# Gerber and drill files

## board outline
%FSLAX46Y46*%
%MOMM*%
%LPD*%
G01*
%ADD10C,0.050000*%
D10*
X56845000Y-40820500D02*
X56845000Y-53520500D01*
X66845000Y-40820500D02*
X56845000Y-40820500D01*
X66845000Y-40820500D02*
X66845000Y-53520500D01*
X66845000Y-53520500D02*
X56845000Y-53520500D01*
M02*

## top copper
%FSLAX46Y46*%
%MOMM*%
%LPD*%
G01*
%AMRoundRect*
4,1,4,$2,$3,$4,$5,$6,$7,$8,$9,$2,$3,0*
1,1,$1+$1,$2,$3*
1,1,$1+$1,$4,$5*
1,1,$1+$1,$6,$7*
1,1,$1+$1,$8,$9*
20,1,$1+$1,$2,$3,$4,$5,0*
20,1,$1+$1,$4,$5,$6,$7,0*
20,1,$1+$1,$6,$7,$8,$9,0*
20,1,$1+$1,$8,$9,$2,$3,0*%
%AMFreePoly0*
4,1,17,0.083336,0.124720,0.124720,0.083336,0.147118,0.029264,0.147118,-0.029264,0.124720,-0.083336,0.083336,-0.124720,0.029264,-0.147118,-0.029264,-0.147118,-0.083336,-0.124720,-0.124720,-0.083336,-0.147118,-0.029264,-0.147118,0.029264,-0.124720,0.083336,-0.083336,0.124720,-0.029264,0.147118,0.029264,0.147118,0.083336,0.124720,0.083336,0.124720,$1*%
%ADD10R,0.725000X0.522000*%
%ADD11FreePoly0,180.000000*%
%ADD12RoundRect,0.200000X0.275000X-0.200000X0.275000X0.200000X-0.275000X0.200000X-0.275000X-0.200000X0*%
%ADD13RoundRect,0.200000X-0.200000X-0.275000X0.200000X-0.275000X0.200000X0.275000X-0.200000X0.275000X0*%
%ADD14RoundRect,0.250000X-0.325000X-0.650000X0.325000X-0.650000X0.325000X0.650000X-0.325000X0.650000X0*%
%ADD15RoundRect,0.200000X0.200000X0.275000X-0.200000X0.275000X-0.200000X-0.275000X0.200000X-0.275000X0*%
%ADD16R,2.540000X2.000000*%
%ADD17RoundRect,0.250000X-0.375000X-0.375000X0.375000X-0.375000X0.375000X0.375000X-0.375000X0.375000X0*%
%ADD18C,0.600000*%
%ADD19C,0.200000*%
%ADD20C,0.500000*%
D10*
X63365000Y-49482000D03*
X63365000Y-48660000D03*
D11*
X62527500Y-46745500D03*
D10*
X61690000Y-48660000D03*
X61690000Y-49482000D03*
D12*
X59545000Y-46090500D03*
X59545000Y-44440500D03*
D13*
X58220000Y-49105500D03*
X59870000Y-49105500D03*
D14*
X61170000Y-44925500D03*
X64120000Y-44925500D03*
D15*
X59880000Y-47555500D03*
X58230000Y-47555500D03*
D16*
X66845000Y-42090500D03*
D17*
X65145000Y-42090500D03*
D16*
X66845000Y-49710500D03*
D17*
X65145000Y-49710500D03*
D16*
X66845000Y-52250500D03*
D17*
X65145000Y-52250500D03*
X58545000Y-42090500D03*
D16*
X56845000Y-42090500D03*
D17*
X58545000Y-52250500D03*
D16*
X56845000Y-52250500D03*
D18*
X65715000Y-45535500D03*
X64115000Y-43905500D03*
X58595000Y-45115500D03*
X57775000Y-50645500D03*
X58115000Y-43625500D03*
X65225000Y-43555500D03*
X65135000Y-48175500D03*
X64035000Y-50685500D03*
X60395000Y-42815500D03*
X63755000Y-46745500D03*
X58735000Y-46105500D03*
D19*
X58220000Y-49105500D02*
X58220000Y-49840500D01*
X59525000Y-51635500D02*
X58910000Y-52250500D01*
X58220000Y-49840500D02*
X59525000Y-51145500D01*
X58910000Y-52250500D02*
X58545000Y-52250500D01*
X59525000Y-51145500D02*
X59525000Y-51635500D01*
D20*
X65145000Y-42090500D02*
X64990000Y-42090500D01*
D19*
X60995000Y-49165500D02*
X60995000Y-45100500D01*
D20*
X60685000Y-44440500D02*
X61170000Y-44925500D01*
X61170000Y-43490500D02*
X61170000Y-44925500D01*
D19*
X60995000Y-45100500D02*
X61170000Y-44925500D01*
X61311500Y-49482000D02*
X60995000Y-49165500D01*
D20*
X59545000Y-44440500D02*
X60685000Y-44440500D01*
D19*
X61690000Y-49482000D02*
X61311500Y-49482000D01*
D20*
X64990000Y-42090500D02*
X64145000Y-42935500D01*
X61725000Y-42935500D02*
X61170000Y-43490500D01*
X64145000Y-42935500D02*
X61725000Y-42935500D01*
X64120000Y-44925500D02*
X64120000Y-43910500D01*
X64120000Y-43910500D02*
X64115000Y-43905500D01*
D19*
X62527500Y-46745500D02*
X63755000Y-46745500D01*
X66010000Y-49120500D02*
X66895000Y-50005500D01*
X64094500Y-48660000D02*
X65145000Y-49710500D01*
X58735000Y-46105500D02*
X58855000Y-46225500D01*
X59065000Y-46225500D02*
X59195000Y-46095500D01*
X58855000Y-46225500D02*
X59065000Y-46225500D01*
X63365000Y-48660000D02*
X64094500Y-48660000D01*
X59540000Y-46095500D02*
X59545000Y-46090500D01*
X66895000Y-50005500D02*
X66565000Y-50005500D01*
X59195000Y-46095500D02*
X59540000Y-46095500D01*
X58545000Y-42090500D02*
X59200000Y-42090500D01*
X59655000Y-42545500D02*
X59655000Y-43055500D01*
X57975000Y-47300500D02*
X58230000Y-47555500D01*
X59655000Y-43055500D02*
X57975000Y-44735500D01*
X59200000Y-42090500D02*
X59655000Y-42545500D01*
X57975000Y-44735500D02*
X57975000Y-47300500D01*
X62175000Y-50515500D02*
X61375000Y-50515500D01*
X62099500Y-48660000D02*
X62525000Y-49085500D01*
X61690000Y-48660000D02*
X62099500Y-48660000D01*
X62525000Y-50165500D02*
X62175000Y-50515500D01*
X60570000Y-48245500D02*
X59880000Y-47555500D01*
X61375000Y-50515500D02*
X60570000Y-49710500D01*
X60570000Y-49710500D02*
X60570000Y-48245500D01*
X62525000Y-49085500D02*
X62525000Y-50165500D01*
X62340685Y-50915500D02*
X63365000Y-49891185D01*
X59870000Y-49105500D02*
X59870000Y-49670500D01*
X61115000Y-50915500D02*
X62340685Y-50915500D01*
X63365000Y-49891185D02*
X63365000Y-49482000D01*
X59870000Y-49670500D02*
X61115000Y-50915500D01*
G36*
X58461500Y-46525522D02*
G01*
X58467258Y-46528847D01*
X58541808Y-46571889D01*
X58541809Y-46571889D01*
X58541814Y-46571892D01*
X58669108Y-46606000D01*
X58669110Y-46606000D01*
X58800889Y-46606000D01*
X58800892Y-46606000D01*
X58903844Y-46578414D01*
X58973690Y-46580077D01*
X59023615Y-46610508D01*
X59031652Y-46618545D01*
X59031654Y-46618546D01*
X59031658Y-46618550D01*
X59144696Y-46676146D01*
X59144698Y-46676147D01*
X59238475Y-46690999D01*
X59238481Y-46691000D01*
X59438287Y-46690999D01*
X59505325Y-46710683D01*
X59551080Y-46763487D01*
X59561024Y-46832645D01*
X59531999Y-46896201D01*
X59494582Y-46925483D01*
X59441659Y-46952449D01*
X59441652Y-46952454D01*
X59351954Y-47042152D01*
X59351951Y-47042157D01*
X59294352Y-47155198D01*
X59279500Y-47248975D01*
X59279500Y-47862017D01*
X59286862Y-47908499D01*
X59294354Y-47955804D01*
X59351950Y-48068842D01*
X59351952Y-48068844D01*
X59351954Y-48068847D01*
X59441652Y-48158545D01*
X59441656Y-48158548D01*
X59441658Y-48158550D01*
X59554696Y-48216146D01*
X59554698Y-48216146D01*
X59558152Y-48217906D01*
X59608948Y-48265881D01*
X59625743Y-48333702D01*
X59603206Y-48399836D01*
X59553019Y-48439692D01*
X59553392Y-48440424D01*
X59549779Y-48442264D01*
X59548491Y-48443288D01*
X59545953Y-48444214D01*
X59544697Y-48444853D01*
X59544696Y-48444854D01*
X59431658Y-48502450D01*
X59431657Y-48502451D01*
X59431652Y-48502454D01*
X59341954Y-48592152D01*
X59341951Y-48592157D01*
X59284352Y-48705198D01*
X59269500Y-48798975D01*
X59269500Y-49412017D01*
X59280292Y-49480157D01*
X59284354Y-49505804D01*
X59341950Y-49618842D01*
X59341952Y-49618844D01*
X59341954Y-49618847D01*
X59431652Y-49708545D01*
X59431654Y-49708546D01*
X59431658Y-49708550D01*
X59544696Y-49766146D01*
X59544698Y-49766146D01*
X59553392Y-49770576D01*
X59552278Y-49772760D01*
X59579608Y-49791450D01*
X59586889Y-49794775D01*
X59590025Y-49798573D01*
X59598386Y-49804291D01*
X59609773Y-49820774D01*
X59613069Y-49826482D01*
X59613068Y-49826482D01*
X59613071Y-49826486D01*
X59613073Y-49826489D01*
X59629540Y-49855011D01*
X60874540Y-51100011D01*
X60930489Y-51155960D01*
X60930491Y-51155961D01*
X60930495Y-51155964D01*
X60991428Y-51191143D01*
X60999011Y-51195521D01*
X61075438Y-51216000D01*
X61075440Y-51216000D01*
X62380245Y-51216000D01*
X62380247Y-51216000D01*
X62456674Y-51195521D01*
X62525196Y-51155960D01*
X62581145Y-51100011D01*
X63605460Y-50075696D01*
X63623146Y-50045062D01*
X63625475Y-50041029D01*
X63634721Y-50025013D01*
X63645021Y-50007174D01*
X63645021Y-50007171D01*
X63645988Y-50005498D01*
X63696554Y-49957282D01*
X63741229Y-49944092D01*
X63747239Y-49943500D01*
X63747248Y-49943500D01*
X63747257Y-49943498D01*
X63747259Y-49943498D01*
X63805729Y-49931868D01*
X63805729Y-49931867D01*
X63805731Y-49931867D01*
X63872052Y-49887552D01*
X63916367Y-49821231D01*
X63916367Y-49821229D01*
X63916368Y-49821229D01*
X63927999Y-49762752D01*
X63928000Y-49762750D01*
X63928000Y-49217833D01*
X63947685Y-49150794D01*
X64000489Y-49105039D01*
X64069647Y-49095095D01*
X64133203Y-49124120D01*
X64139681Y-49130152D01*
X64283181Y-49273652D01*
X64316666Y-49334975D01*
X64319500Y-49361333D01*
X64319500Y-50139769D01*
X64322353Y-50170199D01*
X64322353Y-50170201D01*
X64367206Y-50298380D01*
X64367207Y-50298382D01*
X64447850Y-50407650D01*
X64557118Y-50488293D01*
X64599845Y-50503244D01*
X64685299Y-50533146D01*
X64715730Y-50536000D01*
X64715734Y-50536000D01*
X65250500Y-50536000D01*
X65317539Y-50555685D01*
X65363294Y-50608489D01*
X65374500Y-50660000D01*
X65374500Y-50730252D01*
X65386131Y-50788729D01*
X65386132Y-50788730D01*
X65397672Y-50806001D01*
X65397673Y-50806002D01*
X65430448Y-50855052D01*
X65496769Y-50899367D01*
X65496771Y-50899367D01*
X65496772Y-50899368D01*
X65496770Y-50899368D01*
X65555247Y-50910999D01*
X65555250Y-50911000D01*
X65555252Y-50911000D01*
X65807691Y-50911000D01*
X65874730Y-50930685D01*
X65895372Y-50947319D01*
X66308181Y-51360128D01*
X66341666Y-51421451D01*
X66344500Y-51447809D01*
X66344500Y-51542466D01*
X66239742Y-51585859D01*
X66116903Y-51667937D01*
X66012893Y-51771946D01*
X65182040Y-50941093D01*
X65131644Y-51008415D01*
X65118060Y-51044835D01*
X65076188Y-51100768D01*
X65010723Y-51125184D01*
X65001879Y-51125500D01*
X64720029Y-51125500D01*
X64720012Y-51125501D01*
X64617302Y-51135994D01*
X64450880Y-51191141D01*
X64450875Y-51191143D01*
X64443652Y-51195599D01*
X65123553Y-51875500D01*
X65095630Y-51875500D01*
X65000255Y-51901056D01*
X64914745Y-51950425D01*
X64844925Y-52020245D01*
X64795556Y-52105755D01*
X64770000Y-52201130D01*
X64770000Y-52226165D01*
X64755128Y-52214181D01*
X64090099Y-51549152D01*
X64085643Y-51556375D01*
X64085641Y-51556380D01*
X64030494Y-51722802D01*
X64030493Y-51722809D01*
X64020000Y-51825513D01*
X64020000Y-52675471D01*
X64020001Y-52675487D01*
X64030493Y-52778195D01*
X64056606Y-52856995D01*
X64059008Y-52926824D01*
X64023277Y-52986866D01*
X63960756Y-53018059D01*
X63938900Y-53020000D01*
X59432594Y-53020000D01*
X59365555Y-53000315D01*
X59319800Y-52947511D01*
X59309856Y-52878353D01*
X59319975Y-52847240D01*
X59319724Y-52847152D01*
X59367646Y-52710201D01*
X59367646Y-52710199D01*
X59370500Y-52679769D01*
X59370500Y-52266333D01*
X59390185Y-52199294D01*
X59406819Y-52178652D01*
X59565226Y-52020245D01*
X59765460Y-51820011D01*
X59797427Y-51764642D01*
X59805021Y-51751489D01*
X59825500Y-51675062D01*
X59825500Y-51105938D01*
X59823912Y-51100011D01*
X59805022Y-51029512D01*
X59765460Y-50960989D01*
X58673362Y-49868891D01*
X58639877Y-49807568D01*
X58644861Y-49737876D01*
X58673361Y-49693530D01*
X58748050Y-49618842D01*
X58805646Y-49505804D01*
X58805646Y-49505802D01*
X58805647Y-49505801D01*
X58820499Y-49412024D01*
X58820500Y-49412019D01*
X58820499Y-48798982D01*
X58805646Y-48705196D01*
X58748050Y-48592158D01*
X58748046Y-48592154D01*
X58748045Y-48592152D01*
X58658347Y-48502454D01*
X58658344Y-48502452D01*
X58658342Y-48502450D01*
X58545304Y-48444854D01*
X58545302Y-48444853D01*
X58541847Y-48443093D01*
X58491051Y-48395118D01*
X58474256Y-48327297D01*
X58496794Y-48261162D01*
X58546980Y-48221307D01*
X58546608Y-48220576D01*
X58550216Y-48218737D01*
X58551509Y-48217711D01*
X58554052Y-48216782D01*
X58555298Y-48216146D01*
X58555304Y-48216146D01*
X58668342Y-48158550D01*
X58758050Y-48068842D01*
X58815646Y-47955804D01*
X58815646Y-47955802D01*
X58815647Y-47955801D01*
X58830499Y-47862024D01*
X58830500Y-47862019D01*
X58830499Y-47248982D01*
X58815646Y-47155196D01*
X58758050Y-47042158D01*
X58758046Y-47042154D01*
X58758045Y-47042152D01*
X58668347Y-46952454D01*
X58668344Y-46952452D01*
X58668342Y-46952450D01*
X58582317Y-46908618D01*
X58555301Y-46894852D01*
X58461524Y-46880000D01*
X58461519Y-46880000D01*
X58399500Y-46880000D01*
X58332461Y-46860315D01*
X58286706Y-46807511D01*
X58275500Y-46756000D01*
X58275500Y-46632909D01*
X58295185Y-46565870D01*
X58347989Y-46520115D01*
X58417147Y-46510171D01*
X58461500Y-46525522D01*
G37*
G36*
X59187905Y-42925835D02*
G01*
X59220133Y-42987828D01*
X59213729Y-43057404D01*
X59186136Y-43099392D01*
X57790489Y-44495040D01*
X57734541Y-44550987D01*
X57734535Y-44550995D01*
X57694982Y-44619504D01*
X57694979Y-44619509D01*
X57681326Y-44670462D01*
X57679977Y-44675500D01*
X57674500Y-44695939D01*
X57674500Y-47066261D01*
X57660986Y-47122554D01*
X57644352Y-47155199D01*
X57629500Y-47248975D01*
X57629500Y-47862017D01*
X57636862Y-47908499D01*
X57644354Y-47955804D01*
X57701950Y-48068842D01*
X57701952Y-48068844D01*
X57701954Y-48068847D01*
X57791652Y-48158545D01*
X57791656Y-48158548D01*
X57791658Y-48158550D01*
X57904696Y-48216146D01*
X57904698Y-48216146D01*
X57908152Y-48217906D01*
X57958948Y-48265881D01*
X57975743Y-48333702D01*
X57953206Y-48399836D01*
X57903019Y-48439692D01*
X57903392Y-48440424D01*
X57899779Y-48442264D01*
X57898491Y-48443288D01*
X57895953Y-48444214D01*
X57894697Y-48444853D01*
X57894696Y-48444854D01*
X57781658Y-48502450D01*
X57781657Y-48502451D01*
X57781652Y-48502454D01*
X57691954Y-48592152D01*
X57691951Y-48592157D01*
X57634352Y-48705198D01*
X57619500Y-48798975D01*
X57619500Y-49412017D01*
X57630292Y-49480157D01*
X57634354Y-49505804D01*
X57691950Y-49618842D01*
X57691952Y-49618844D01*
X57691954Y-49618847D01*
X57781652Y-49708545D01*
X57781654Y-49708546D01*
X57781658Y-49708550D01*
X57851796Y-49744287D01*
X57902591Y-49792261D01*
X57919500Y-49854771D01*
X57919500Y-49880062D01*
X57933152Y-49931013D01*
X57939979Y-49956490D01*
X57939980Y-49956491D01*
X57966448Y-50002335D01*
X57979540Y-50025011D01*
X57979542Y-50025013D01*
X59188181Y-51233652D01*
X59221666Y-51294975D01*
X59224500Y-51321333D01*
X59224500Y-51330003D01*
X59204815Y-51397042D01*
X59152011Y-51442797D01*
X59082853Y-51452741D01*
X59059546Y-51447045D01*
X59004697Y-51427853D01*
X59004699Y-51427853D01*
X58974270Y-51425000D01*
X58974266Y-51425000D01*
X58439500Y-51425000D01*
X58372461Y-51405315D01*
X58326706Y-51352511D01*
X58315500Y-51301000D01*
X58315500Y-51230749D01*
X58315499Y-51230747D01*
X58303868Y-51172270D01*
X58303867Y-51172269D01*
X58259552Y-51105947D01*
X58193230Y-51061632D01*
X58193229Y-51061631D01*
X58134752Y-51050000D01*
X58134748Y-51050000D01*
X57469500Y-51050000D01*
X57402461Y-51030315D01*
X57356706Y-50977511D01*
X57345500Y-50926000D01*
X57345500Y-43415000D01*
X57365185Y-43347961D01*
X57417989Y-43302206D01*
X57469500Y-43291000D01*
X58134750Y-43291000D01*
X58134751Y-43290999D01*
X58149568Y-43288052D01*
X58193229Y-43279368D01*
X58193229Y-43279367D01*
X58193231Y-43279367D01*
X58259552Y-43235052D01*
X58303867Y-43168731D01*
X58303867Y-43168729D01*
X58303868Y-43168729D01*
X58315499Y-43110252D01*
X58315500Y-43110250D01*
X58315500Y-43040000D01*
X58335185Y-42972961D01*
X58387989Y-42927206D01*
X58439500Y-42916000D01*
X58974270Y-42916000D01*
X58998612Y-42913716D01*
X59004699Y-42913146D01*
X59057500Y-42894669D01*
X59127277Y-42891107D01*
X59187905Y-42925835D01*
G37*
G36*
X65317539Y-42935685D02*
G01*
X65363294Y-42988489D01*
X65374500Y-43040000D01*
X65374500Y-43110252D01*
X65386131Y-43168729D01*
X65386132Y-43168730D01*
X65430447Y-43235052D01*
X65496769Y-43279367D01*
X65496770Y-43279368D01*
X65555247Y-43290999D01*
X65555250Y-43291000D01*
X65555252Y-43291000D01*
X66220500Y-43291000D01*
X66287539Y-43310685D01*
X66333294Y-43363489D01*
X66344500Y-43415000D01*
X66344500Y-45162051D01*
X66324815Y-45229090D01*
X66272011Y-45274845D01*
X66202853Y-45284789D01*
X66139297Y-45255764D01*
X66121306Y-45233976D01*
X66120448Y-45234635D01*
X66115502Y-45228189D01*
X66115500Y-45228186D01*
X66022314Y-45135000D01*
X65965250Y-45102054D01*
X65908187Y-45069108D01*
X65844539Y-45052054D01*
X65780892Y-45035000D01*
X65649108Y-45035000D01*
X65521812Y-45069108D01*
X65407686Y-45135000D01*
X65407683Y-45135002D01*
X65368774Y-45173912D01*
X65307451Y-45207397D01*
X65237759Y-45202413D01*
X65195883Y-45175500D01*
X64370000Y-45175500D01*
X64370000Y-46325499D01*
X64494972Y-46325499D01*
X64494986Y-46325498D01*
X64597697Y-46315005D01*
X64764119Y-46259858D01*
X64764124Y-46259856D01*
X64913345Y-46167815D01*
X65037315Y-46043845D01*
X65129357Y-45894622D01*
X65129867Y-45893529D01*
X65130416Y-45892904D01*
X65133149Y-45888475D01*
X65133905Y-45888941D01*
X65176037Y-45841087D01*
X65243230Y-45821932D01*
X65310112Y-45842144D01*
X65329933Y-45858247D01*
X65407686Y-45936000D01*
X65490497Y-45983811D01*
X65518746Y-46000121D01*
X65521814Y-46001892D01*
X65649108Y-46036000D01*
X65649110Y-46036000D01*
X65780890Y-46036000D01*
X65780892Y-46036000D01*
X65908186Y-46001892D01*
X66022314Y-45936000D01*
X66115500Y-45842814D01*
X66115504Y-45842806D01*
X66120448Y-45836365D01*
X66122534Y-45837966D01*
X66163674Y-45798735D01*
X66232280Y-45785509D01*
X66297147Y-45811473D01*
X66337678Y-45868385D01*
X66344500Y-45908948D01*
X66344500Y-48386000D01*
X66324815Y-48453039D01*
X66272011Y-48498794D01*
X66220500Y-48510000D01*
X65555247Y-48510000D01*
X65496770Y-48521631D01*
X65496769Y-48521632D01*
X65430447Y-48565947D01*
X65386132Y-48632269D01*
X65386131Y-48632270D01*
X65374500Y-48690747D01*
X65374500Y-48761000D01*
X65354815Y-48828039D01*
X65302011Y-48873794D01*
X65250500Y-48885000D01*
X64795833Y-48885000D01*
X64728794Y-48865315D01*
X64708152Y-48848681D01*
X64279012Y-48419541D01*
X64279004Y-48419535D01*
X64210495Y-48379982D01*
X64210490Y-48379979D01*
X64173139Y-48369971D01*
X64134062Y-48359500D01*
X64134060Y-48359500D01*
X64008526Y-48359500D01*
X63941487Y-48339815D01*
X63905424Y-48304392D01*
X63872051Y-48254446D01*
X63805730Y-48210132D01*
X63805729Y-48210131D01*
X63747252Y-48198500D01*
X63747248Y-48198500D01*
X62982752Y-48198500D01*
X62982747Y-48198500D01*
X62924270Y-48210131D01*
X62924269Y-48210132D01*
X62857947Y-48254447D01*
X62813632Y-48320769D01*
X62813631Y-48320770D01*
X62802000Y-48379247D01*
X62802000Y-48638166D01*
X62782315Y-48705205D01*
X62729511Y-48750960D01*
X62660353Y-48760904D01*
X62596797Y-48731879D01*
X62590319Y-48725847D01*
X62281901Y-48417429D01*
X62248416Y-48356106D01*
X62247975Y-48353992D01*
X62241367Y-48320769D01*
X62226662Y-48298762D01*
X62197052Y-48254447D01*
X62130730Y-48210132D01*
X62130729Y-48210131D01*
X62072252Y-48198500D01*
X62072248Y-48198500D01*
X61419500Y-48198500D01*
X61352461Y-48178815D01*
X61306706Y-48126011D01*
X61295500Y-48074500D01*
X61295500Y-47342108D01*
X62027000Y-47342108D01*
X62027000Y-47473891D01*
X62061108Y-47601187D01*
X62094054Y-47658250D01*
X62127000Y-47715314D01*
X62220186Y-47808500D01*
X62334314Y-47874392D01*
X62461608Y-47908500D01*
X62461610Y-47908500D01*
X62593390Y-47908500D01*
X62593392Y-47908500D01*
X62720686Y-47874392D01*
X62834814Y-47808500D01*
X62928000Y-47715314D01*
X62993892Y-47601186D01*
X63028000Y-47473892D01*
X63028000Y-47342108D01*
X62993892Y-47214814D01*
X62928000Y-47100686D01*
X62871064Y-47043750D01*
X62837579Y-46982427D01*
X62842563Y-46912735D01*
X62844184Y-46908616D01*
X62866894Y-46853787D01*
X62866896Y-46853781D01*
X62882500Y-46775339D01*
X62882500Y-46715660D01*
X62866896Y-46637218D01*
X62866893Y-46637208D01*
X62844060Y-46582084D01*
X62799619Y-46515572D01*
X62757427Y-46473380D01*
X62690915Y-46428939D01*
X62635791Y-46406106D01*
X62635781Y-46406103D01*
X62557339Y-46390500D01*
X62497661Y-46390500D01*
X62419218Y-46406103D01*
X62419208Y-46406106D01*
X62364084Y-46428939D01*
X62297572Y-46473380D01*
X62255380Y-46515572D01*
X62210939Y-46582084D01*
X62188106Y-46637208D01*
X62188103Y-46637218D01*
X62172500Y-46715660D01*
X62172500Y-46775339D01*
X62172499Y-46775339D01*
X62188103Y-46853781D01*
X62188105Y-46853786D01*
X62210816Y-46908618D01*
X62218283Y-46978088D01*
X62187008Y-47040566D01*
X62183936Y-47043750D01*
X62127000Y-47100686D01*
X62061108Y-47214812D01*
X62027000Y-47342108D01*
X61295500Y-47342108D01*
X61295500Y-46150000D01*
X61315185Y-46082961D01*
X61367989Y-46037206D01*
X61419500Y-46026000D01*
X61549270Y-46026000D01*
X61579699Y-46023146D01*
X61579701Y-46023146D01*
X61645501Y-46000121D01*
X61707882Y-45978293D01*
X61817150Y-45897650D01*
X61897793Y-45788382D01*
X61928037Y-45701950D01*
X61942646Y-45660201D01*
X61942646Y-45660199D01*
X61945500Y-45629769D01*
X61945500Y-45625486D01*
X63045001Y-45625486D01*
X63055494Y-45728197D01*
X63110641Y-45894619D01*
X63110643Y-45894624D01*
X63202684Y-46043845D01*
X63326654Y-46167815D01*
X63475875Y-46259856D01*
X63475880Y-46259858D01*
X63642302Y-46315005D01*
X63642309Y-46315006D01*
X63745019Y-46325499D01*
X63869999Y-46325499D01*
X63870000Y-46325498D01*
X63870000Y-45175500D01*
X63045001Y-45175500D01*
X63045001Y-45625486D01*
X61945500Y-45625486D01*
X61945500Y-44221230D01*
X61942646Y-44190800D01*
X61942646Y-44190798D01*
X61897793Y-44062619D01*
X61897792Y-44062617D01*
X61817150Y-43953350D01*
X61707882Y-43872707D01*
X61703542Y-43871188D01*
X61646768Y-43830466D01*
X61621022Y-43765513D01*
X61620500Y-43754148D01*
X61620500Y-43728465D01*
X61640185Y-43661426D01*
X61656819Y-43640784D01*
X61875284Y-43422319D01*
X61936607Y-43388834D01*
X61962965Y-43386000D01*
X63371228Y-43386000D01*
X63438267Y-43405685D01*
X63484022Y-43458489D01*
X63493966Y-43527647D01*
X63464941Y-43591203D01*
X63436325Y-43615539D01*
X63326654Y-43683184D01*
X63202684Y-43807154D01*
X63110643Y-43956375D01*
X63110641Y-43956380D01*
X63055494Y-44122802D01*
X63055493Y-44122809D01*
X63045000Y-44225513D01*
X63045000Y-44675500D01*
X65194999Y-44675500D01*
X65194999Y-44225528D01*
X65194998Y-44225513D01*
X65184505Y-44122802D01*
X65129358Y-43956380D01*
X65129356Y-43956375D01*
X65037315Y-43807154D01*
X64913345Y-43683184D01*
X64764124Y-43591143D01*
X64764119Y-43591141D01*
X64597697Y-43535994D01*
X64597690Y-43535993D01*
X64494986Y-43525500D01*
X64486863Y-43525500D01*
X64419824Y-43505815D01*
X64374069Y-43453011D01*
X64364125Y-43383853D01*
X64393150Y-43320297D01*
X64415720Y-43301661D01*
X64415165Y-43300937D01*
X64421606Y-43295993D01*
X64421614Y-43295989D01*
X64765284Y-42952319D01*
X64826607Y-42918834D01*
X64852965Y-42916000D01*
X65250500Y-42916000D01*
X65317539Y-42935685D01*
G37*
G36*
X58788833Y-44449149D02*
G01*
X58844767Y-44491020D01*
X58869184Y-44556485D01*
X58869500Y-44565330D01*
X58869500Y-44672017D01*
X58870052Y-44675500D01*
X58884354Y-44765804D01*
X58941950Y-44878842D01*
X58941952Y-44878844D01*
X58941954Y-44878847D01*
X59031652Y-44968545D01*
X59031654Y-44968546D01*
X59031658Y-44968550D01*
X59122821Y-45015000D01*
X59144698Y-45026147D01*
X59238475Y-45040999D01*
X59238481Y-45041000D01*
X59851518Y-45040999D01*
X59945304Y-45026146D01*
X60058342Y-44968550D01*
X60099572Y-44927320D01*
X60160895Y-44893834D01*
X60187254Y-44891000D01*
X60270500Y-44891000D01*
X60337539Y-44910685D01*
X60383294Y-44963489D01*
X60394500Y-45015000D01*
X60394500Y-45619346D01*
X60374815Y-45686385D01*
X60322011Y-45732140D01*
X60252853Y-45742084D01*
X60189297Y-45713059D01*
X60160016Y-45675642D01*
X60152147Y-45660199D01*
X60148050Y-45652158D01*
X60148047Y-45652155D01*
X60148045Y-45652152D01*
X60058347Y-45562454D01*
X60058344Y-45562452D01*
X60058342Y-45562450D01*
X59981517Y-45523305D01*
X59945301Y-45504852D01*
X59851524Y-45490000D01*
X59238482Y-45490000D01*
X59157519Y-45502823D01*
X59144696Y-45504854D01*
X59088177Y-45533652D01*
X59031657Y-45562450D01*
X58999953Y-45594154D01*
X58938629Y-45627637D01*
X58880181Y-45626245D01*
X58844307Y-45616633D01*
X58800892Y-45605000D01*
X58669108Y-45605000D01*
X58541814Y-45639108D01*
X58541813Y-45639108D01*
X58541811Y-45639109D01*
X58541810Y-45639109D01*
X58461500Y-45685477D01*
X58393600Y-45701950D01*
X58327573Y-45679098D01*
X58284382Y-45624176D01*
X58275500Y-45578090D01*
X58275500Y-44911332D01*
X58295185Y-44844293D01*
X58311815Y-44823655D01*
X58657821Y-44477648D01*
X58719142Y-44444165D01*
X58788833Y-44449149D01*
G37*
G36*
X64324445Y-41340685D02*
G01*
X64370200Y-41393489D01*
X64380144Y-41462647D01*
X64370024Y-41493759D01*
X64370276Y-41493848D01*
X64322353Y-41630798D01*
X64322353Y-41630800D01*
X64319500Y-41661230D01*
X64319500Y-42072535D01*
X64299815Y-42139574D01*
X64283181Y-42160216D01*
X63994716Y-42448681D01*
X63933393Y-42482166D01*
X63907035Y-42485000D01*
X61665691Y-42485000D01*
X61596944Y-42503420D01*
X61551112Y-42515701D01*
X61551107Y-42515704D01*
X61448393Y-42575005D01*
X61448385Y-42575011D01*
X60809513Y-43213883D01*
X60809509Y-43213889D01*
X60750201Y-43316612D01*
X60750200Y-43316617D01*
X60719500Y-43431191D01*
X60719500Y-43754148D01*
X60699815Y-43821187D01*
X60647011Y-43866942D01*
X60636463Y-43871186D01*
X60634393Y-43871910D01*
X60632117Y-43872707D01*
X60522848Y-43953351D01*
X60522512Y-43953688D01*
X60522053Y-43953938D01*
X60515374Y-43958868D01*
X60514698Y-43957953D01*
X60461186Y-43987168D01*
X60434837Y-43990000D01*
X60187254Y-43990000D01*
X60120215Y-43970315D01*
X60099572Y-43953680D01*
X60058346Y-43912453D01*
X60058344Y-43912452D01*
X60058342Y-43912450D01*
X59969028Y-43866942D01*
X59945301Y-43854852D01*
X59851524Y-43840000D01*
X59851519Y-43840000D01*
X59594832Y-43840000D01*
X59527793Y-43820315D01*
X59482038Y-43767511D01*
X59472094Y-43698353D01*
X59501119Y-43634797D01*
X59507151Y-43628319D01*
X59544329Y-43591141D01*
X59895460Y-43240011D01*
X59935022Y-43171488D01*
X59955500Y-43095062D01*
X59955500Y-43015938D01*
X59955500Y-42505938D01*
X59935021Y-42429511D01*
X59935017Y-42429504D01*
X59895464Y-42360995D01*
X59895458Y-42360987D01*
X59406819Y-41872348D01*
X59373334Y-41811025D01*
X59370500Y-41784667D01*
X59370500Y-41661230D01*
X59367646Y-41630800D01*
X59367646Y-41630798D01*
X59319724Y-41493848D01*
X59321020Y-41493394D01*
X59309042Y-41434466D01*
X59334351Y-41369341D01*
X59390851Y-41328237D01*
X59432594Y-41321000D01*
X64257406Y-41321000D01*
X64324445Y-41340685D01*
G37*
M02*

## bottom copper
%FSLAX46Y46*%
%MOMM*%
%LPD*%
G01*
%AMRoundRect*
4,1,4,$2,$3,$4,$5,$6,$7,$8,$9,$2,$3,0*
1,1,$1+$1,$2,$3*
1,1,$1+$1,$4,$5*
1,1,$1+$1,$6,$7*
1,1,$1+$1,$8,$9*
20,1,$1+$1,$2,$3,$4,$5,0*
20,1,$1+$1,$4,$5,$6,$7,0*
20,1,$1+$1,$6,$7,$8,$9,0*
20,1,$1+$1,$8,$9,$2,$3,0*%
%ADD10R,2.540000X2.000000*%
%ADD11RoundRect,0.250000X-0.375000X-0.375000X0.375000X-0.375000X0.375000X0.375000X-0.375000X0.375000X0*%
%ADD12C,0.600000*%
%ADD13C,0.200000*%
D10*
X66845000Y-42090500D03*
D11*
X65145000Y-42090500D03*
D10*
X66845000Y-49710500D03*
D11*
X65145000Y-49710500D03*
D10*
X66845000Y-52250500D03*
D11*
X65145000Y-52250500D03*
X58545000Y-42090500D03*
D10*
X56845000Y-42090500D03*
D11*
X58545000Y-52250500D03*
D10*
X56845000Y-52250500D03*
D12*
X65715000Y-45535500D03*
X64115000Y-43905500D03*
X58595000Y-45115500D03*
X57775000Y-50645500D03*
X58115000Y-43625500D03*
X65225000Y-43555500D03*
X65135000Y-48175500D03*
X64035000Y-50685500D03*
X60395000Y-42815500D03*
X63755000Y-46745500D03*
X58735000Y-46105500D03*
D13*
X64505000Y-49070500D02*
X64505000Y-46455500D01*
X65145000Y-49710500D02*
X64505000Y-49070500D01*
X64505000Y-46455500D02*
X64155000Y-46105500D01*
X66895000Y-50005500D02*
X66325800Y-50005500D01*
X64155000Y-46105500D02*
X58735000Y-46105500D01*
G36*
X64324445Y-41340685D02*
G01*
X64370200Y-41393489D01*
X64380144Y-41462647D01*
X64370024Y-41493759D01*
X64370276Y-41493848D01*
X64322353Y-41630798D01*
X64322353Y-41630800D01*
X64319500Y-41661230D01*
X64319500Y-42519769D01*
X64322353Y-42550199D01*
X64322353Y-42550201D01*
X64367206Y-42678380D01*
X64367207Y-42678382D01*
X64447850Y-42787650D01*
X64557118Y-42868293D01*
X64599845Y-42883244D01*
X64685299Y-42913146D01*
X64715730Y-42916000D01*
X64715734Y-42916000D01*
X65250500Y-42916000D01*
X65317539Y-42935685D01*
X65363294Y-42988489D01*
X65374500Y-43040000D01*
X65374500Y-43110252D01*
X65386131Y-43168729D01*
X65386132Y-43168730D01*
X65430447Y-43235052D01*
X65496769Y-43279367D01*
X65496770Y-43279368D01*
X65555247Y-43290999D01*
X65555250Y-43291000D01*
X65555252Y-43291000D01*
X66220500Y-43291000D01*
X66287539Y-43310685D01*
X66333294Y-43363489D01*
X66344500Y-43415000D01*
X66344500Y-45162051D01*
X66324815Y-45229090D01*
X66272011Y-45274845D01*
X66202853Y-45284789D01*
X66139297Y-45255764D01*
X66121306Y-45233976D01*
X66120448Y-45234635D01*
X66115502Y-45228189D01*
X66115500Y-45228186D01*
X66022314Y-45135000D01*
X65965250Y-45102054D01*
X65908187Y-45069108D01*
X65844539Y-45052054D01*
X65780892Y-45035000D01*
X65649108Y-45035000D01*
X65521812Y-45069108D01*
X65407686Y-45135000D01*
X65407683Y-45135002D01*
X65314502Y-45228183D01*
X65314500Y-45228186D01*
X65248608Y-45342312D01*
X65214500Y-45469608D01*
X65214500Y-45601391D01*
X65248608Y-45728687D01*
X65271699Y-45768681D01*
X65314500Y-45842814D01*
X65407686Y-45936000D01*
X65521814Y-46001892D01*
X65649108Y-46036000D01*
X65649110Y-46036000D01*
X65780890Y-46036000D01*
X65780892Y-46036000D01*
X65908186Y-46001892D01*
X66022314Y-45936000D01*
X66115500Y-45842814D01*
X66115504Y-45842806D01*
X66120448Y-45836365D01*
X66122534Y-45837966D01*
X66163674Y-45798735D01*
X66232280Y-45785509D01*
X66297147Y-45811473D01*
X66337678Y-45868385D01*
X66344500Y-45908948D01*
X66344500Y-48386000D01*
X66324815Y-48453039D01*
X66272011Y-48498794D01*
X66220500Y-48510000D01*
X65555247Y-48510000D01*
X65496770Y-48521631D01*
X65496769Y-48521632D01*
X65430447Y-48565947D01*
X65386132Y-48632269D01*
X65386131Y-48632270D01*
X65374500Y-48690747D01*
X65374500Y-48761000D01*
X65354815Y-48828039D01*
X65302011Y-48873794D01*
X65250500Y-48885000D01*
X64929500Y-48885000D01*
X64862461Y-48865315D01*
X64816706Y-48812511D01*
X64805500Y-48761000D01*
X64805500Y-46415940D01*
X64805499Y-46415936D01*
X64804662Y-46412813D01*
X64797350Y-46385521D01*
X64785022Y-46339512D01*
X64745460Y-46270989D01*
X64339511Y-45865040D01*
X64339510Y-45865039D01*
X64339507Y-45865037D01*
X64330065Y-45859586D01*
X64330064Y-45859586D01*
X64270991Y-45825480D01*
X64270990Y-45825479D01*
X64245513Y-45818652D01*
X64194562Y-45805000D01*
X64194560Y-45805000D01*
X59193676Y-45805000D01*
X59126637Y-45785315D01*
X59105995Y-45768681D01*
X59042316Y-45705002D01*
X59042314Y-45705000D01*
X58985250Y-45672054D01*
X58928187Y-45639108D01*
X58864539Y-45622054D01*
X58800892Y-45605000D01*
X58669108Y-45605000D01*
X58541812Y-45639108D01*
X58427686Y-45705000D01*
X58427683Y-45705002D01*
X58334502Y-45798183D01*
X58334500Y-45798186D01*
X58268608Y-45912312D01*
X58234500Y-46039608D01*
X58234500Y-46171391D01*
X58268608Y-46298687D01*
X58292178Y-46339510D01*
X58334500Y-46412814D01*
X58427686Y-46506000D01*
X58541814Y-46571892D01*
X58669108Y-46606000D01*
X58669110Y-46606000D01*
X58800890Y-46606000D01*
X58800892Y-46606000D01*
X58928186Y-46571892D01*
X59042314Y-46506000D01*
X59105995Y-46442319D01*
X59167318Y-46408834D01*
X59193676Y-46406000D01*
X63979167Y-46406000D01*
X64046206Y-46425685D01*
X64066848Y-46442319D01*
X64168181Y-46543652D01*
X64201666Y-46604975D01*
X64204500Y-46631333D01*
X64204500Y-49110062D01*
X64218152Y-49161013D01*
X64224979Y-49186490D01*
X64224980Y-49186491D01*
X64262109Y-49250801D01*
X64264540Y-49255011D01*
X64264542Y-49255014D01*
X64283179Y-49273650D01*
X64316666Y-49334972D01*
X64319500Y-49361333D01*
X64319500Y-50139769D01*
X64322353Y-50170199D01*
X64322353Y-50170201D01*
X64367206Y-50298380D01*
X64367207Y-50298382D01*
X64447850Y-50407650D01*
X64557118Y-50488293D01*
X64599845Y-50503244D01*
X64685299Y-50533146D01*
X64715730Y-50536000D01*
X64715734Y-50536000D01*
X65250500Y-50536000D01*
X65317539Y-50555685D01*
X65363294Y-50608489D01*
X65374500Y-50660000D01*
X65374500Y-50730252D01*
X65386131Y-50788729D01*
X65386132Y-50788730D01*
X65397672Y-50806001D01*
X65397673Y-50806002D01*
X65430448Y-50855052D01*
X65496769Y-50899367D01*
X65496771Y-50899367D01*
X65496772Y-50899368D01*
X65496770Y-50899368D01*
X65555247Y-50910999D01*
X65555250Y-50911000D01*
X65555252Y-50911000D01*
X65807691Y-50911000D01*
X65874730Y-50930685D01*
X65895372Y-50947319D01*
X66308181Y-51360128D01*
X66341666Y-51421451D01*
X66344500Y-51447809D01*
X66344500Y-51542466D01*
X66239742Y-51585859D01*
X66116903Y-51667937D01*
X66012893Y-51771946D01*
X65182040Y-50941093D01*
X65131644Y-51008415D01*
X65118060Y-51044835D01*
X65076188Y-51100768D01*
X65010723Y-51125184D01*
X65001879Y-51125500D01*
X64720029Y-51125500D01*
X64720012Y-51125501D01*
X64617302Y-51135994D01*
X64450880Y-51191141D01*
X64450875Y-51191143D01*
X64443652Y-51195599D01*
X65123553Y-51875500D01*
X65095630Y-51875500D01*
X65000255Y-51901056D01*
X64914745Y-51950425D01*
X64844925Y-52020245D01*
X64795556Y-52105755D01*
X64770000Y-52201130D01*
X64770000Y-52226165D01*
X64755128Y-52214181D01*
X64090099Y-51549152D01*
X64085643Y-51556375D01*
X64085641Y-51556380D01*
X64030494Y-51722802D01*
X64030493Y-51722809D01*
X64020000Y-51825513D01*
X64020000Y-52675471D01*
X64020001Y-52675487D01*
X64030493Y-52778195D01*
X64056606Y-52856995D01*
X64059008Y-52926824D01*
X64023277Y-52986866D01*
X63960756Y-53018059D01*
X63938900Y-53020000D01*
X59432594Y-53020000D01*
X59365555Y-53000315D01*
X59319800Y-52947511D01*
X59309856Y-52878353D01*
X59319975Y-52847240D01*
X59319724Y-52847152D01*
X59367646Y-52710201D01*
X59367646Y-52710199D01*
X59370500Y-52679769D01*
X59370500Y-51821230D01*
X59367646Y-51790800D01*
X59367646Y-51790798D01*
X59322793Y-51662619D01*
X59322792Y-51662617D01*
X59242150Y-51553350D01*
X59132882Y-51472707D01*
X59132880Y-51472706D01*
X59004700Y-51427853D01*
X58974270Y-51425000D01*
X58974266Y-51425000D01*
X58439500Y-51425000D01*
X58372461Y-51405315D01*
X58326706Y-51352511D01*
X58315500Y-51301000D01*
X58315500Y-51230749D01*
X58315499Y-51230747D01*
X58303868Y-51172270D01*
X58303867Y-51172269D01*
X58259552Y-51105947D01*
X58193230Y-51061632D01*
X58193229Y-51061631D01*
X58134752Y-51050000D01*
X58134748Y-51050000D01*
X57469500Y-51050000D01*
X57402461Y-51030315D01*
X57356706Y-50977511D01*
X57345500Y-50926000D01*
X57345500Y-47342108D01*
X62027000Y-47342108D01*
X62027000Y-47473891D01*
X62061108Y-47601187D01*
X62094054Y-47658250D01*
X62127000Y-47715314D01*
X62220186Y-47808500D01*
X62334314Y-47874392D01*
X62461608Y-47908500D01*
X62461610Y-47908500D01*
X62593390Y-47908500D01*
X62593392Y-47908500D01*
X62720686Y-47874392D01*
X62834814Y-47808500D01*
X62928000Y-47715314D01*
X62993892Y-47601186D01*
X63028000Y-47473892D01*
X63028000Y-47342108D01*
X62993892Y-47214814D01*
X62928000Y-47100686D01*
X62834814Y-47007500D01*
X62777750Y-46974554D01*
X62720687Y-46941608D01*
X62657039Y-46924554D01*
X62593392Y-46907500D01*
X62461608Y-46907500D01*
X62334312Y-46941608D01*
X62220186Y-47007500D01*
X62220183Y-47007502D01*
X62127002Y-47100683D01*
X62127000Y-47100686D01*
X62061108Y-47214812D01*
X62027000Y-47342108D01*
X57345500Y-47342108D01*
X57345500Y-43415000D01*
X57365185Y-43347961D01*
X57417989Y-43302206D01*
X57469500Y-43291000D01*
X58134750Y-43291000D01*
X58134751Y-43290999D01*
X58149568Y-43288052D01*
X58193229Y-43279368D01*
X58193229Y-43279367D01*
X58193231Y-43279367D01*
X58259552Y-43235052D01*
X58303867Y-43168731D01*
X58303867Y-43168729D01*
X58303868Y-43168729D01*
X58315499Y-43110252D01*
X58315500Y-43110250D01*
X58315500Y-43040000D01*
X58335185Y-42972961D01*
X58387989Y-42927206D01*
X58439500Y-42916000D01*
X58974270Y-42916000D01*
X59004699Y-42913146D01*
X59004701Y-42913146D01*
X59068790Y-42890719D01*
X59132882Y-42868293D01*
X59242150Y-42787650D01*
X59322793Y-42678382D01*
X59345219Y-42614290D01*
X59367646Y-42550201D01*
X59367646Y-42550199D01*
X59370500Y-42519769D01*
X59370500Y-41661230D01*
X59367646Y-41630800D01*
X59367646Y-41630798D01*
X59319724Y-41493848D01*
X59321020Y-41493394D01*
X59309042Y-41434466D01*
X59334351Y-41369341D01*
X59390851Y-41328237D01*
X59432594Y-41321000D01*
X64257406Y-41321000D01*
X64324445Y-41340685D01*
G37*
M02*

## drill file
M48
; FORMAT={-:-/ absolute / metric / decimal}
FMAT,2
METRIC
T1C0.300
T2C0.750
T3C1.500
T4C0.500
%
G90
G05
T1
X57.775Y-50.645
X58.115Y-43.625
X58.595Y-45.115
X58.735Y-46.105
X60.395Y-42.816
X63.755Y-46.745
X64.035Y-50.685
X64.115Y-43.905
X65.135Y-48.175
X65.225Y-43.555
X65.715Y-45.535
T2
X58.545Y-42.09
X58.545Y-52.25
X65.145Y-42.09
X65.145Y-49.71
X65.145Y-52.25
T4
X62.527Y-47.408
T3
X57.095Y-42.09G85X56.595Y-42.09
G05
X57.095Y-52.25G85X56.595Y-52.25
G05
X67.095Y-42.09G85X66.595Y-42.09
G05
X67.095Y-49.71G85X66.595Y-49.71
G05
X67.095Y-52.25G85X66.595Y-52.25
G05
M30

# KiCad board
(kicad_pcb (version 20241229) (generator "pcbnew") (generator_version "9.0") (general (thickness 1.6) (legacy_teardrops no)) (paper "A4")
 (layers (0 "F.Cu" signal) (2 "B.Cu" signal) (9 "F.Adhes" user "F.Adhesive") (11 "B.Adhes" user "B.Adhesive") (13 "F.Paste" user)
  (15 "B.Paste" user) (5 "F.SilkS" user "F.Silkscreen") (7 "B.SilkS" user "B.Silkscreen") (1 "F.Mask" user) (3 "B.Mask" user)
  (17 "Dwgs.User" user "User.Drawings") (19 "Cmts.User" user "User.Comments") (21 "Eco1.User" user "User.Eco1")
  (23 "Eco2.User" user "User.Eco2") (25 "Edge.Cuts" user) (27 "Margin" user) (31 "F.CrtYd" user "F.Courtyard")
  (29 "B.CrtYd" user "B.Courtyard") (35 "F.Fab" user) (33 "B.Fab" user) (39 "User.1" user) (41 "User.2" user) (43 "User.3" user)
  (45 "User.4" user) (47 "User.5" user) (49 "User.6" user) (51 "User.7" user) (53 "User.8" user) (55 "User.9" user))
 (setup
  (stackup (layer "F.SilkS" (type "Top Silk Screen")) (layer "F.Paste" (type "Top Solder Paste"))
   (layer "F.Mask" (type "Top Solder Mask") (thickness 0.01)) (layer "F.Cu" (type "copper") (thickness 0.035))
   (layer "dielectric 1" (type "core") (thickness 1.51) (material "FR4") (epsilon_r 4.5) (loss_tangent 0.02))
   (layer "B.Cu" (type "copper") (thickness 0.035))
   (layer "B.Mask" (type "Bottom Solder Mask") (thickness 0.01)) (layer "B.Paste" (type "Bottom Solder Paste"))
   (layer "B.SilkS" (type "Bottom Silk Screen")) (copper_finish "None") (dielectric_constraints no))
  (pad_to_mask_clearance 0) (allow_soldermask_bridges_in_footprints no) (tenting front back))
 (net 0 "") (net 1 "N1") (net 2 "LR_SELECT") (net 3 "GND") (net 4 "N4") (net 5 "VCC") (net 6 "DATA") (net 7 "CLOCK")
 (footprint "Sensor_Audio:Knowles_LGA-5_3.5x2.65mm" (layer "F.Cu") (at 62.5275 48.178 180)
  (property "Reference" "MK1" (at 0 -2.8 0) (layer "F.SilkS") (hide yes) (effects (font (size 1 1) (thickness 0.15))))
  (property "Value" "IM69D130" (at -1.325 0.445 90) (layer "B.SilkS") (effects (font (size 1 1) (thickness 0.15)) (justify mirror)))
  (pad "" np_thru_hole circle (at 0 0.77 180) (size 0.5 0.5) (drill 0.5) (layers "*.Cu" "*.Mask"))
  (pad "1" smd rect (at -0.8375 -1.304 180) (size 0.725 0.522) (layers "F.Cu" "F.Mask" "F.Paste") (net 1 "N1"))
  (pad "2" smd rect (at -0.8375 -0.482 180) (size 0.725 0.522) (layers "F.Cu" "F.Mask" "F.Paste") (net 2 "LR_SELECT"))
  (pad "3" smd custom (at 0 1.4325 180) (size 0.3 0.3) (layers "F.Cu" "F.Mask") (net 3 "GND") (zone_connect 0)
   (options (clearance outline) (anchor circle)) (primitives))
  (pad "4" smd rect (at 0.8375 -0.482 180) (size 0.725 0.522) (layers "F.Cu" "F.Mask" "F.Paste") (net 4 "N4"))
  (pad "5" smd rect (at 0.8375 -1.304 180) (size 0.725 0.522) (layers "F.Cu" "F.Mask" "F.Paste") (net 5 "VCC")))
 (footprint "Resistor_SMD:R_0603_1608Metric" (layer "F.Cu") (at 59.545 45.2655 90)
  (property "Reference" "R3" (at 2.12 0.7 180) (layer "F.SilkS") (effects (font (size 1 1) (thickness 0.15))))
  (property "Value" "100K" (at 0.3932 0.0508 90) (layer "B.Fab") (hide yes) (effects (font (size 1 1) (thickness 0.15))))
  (pad "1" smd roundrect (at -0.825 0 90) (size 0.8 0.95) (layers "F.Cu" "F.Mask" "F.Paste") (roundrect_rratio 0.25) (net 2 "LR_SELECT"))
  (pad "2" smd roundrect (at 0.825 0 90) (size 0.8 0.95) (layers "F.Cu" "F.Mask" "F.Paste") (roundrect_rratio 0.25) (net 5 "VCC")))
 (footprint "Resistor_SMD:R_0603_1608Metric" (layer "F.Cu") (at 59.045 49.1055)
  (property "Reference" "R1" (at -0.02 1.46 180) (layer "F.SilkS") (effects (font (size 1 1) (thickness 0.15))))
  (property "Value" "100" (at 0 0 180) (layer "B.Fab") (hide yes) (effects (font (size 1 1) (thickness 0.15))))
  (pad "1" smd roundrect (at -0.825 0) (size 0.8 0.95) (layers "F.Cu" "F.Mask" "F.Paste") (roundrect_rratio 0.25) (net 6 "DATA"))
  (pad "2" smd roundrect (at 0.825 0) (size 0.8 0.95) (layers "F.Cu" "F.Mask" "F.Paste") (roundrect_rratio 0.25) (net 1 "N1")))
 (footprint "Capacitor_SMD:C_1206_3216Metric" (layer "F.Cu") (at 62.645 44.9255)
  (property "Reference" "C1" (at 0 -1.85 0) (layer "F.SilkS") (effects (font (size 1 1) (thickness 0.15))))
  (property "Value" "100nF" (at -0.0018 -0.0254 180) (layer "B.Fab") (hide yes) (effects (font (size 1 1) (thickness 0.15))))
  (pad "1" smd roundrect (at -1.475 0) (size 1.15 1.8) (layers "F.Cu" "F.Mask" "F.Paste") (roundrect_rratio 0.217391) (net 5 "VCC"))
  (pad "2" smd roundrect (at 1.475 0) (size 1.15 1.8) (layers "F.Cu" "F.Mask" "F.Paste") (roundrect_rratio 0.217391) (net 3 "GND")))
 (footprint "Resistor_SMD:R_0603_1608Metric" (layer "F.Cu") (at 59.055 47.5555 180)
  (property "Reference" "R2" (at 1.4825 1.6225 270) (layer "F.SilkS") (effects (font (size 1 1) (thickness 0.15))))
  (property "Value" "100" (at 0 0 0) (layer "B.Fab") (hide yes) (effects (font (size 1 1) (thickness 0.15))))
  (pad "1" smd roundrect (at -0.825 0 180) (size 0.8 0.95) (layers "F.Cu" "F.Mask" "F.Paste") (roundrect_rratio 0.25) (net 4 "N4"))
  (pad "2" smd roundrect (at 0.825 0 180) (size 0.8 0.95) (layers "F.Cu" "F.Mask" "F.Paste") (roundrect_rratio 0.25) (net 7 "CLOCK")))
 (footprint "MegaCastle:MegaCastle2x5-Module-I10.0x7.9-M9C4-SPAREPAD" (layer "B.Cu") (at 61.845 47.1705 180)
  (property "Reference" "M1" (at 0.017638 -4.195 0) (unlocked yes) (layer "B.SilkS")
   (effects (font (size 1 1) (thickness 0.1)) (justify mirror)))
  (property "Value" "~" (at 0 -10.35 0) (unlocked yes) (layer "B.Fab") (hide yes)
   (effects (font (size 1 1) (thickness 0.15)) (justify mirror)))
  (fp_line (start 5 6.35) (end 5 -6.35) (stroke (width 0.05) (type default)) (layer "Edge.Cuts"))
  (fp_line (start -5 6.35) (end 5 6.35) (stroke (width 0.05) (type default)) (layer "Edge.Cuts"))
  (fp_line (start -5 6.35) (end -5 -6.35) (stroke (width 0.05) (type default)) (layer "Edge.Cuts"))
  (fp_line (start -5 -6.35) (end 5 -6.35) (stroke (width 0.05) (type default)) (layer "Edge.Cuts"))
  (pad "1" thru_hole rect (at -5 5.08 180) (size 2.54 2) (drill oval 2 1.5) (layers "*.Cu" "*.Mask") (remove_unused_layers no) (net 5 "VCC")
   (thermal_bridge_angle 45))
  (pad "1" thru_hole roundrect (at -3.3 5.08) (size 1.25 1.25) (drill 0.75) (layers "*.Cu" "*.Mask") (remove_unused_layers no)
   (roundrect_rratio 0.2) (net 5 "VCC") (thermal_bridge_angle 45))
  (pad "4" thru_hole rect (at -5 -2.54 180) (size 2.54 2) (drill oval 2 1.5) (layers "*.Cu" "*.Mask") (remove_unused_layers no)
   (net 2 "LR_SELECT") (thermal_bridge_angle 45))
  (pad "4" thru_hole roundrect (at -3.3 -2.54) (size 1.25 1.25) (drill 0.75) (layers "*.Cu" "*.Mask") (remove_unused_layers no)
   (roundrect_rratio 0.2) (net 2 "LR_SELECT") (thermal_bridge_angle 45))
  (pad "5" thru_hole rect (at -5 -5.08 180) (size 2.54 2) (drill oval 2 1.5) (layers "*.Cu" "*.Mask") (remove_unused_layers no)
   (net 3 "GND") (thermal_bridge_angle 45))
  (pad "5" thru_hole roundrect (at -3.3 -5.08) (size 1.25 1.25) (drill 0.75) (layers "*.Cu" "*.Mask") (remove_unused_layers no)
   (roundrect_rratio 0.2) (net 3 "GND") (thermal_bridge_angle 45))
  (pad "6" thru_hole roundrect (at 3.3 5.08) (size 1.25 1.25) (drill 0.75) (layers "*.Cu" "*.Mask") (remove_unused_layers no)
   (roundrect_rratio 0.2) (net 7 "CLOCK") (thermal_bridge_angle 45))
  (pad "6" thru_hole rect (at 5 5.08 180) (size 2.54 2) (drill oval 2 1.5) (layers "*.Cu" "*.Mask") (remove_unused_layers no)
   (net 7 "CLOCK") (thermal_bridge_angle 45))
  (pad "10" thru_hole roundrect (at 3.3 -5.08) (size 1.25 1.25) (drill 0.75) (layers "*.Cu" "*.Mask") (remove_unused_layers no)
   (roundrect_rratio 0.2) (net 6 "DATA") (thermal_bridge_angle 45))
  (pad "10" thru_hole rect (at 5 -5.08 180) (size 2.54 2) (drill oval 2 1.5) (layers "*.Cu" "*.Mask") (remove_unused_layers no)
   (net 6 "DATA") (thermal_bridge_angle 45))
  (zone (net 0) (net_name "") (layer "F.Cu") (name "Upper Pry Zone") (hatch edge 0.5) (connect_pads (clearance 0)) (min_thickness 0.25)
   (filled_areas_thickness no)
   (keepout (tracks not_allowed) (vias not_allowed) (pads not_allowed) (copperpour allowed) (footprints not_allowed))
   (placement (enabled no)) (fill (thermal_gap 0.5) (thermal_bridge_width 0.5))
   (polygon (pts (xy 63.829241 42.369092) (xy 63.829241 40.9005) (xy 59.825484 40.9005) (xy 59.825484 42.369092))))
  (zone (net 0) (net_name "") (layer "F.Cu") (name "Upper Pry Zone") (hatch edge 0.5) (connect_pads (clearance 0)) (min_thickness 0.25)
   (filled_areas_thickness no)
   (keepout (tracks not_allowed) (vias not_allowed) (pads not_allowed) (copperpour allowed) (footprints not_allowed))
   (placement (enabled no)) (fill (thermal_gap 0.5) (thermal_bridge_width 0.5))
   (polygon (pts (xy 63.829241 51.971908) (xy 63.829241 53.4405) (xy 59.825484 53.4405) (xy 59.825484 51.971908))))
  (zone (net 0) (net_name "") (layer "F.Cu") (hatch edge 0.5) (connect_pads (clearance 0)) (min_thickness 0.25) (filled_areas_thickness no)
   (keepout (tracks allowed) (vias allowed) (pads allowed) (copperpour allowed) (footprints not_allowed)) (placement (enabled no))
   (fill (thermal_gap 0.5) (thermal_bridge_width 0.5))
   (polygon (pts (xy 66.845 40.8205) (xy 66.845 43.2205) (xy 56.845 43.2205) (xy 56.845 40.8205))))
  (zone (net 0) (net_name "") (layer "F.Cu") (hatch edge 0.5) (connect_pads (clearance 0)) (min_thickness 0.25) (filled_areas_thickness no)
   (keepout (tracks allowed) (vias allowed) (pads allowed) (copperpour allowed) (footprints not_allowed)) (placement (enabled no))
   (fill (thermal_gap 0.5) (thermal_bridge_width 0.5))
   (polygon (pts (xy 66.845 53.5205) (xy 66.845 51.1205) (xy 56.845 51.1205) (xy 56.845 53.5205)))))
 (via (at 65.715 45.5355) (size 0.6) (drill 0.3) (layers "F.Cu" "B.Cu") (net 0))
 (segment (start 58.22 49.1055) (end 58.22 49.8405) (width 0.2) (layer "F.Cu") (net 6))
 (segment (start 59.525 51.6355) (end 58.91 52.2505) (width 0.2) (layer "F.Cu") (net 6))
 (segment (start 58.22 49.8405) (end 59.525 51.1455) (width 0.2) (layer "F.Cu") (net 6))
 (segment (start 58.91 52.2505) (end 58.545 52.2505) (width 0.2) (layer "F.Cu") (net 6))
 (segment (start 59.525 51.1455) (end 59.525 51.6355) (width 0.2) (layer "F.Cu") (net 6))
 (segment (start 65.145 42.0905) (end 64.99 42.0905) (width 0.5) (layer "F.Cu") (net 5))
 (segment (start 60.995 49.1655) (end 60.995 45.1005) (width 0.2) (layer "F.Cu") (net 5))
 (segment (start 60.685 44.4405) (end 61.17 44.9255) (width 0.5) (layer "F.Cu") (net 5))
 (segment (start 61.17 43.4905) (end 61.17 44.9255) (width 0.5) (layer "F.Cu") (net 5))
 (segment (start 60.995 45.1005) (end 61.17 44.9255) (width 0.2) (layer "F.Cu") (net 5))
 (segment (start 61.3115 49.482) (end 60.995 49.1655) (width 0.2) (layer "F.Cu") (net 5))
 (segment (start 59.545 44.4405) (end 60.685 44.4405) (width 0.5) (layer "F.Cu") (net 5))
 (segment (start 61.69 49.482) (end 61.3115 49.482) (width 0.2) (layer "F.Cu") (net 5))
 (segment (start 64.99 42.0905) (end 64.145 42.9355) (width 0.5) (layer "F.Cu") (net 5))
 (segment (start 61.725 42.9355) (end 61.17 43.4905) (width 0.5) (layer "F.Cu") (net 5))
 (segment (start 64.145 42.9355) (end 61.725 42.9355) (width 0.5) (layer "F.Cu") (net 5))
 (segment (start 64.12 44.9255) (end 64.12 43.9105) (width 0.5) (layer "F.Cu") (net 3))
 (segment (start 64.12 43.9105) (end 64.115 43.9055) (width 0.5) (layer "F.Cu") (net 3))
 (segment (start 62.5275 46.7455) (end 63.755 46.7455) (width 0.2) (layer "F.Cu") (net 3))
 (via (at 64.115 43.9055) (size 0.6) (drill 0.3) (layers "F.Cu" "B.Cu") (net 3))
 (via (at 58.595 45.1155) (size 0.6) (drill 0.3) (layers "F.Cu" "B.Cu") (free yes) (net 3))
 (via (at 57.775 50.6455) (size 0.6) (drill 0.3) (layers "F.Cu" "B.Cu") (free yes) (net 3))
 (via (at 58.115 43.6255) (size 0.6) (drill 0.3) (layers "F.Cu" "B.Cu") (free yes) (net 3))
 (via (at 65.225 43.5555) (size 0.6) (drill 0.3) (layers "F.Cu" "B.Cu") (free yes) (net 3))
 (via (at 65.135 48.1755) (size 0.6) (drill 0.3) (layers "F.Cu" "B.Cu") (free yes) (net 3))
 (via (at 64.035 50.6855) (size 0.6) (drill 0.3) (layers "F.Cu" "B.Cu") (free yes) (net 3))
 (via (at 60.395 42.8155) (size 0.6) (drill 0.3) (layers "F.Cu" "B.Cu") (free yes) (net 3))
 (via (at 63.755 46.7455) (size 0.6) (drill 0.3) (layers "F.Cu" "B.Cu") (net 3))
 (segment (start 66.01 49.1205) (end 66.895 50.0055) (width 0.2) (layer "F.Cu") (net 2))
 (segment (start 64.0945 48.66) (end 65.145 49.7105) (width 0.2) (layer "F.Cu") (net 2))
 (segment (start 58.735 46.1055) (end 58.855 46.2255) (width 0.2) (layer "F.Cu") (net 2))
 (segment (start 59.065 46.2255) (end 59.195 46.0955) (width 0.2) (layer "F.Cu") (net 2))
 (segment (start 58.855 46.2255) (end 59.065 46.2255) (width 0.2) (layer "F.Cu") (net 2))
 (segment (start 63.365 48.66) (end 64.0945 48.66) (width 0.2) (layer "F.Cu") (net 2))
 (segment (start 59.54 46.0955) (end 59.545 46.0905) (width 0.2) (layer "F.Cu") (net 2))
 (segment (start 66.895 50.0055) (end 66.565 50.0055) (width 0.2) (layer "F.Cu") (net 2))
 (segment (start 59.195 46.0955) (end 59.54 46.0955) (width 0.2) (layer "F.Cu") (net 2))
 (via (at 58.735 46.1055) (size 0.6) (drill 0.3) (layers "F.Cu" "B.Cu") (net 2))
 (segment (start 64.505 49.0705) (end 64.505 46.4555) (width 0.2) (layer "B.Cu") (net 2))
 (segment (start 65.145 49.7105) (end 64.505 49.0705) (width 0.2) (layer "B.Cu") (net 2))
 (segment (start 64.505 46.4555) (end 64.155 46.1055) (width 0.2) (layer "B.Cu") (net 2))
 (segment (start 66.895 50.0055) (end 66.3258 50.0055) (width 0.2) (layer "B.Cu") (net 2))
 (segment (start 64.155 46.1055) (end 58.735 46.1055) (width 0.2) (layer "B.Cu") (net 2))
 (segment (start 58.545 42.0905) (end 59.2 42.0905) (width 0.2) (layer "F.Cu") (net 7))
 (segment (start 59.655 42.5455) (end 59.655 43.0555) (width 0.2) (layer "F.Cu") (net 7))
 (segment (start 57.975 47.3005) (end 58.23 47.5555) (width 0.2) (layer "F.Cu") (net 7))
 (segment (start 59.655 43.0555) (end 57.975 44.7355) (width 0.2) (layer "F.Cu") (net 7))
 (segment (start 59.2 42.0905) (end 59.655 42.5455) (width 0.2) (layer "F.Cu") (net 7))
 (segment (start 57.975 44.7355) (end 57.975 47.3005) (width 0.2) (layer "F.Cu") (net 7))
 (segment (start 62.175 50.5155) (end 61.375 50.5155) (width 0.2) (layer "F.Cu") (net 4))
 (segment (start 62.0995 48.66) (end 62.525 49.0855) (width 0.2) (layer "F.Cu") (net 4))
 (segment (start 61.69 48.66) (end 62.0995 48.66) (width 0.2) (layer "F.Cu") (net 4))
 (segment (start 62.525 50.1655) (end 62.175 50.5155) (width 0.2) (layer "F.Cu") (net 4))
 (segment (start 60.57 48.2455) (end 59.88 47.5555) (width 0.2) (layer "F.Cu") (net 4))
 (segment (start 61.375 50.5155) (end 60.57 49.7105) (width 0.2) (layer "F.Cu") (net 4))
 (segment (start 60.57 49.7105) (end 60.57 48.2455) (width 0.2) (layer "F.Cu") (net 4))
 (segment (start 62.525 49.0855) (end 62.525 50.1655) (width 0.2) (layer "F.Cu") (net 4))
 (segment (start 62.340685 50.9155) (end 63.365 49.891185) (width 0.2) (layer "F.Cu") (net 1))
 (segment (start 59.87 49.1055) (end 59.87 49.6705) (width 0.2) (layer "F.Cu") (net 1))
 (segment (start 61.115 50.9155) (end 62.340685 50.9155) (width 0.2) (layer "F.Cu") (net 1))
 (segment (start 63.365 49.891185) (end 63.365 49.482) (width 0.2) (layer "F.Cu") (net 1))
 (segment (start 59.87 49.6705) (end 61.115 50.9155) (width 0.2) (layer "F.Cu") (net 1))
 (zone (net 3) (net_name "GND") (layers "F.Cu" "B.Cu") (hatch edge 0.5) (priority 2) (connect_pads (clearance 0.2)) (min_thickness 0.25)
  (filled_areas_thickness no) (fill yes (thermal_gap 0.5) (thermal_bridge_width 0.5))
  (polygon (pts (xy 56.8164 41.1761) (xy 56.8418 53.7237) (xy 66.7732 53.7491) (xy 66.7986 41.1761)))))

